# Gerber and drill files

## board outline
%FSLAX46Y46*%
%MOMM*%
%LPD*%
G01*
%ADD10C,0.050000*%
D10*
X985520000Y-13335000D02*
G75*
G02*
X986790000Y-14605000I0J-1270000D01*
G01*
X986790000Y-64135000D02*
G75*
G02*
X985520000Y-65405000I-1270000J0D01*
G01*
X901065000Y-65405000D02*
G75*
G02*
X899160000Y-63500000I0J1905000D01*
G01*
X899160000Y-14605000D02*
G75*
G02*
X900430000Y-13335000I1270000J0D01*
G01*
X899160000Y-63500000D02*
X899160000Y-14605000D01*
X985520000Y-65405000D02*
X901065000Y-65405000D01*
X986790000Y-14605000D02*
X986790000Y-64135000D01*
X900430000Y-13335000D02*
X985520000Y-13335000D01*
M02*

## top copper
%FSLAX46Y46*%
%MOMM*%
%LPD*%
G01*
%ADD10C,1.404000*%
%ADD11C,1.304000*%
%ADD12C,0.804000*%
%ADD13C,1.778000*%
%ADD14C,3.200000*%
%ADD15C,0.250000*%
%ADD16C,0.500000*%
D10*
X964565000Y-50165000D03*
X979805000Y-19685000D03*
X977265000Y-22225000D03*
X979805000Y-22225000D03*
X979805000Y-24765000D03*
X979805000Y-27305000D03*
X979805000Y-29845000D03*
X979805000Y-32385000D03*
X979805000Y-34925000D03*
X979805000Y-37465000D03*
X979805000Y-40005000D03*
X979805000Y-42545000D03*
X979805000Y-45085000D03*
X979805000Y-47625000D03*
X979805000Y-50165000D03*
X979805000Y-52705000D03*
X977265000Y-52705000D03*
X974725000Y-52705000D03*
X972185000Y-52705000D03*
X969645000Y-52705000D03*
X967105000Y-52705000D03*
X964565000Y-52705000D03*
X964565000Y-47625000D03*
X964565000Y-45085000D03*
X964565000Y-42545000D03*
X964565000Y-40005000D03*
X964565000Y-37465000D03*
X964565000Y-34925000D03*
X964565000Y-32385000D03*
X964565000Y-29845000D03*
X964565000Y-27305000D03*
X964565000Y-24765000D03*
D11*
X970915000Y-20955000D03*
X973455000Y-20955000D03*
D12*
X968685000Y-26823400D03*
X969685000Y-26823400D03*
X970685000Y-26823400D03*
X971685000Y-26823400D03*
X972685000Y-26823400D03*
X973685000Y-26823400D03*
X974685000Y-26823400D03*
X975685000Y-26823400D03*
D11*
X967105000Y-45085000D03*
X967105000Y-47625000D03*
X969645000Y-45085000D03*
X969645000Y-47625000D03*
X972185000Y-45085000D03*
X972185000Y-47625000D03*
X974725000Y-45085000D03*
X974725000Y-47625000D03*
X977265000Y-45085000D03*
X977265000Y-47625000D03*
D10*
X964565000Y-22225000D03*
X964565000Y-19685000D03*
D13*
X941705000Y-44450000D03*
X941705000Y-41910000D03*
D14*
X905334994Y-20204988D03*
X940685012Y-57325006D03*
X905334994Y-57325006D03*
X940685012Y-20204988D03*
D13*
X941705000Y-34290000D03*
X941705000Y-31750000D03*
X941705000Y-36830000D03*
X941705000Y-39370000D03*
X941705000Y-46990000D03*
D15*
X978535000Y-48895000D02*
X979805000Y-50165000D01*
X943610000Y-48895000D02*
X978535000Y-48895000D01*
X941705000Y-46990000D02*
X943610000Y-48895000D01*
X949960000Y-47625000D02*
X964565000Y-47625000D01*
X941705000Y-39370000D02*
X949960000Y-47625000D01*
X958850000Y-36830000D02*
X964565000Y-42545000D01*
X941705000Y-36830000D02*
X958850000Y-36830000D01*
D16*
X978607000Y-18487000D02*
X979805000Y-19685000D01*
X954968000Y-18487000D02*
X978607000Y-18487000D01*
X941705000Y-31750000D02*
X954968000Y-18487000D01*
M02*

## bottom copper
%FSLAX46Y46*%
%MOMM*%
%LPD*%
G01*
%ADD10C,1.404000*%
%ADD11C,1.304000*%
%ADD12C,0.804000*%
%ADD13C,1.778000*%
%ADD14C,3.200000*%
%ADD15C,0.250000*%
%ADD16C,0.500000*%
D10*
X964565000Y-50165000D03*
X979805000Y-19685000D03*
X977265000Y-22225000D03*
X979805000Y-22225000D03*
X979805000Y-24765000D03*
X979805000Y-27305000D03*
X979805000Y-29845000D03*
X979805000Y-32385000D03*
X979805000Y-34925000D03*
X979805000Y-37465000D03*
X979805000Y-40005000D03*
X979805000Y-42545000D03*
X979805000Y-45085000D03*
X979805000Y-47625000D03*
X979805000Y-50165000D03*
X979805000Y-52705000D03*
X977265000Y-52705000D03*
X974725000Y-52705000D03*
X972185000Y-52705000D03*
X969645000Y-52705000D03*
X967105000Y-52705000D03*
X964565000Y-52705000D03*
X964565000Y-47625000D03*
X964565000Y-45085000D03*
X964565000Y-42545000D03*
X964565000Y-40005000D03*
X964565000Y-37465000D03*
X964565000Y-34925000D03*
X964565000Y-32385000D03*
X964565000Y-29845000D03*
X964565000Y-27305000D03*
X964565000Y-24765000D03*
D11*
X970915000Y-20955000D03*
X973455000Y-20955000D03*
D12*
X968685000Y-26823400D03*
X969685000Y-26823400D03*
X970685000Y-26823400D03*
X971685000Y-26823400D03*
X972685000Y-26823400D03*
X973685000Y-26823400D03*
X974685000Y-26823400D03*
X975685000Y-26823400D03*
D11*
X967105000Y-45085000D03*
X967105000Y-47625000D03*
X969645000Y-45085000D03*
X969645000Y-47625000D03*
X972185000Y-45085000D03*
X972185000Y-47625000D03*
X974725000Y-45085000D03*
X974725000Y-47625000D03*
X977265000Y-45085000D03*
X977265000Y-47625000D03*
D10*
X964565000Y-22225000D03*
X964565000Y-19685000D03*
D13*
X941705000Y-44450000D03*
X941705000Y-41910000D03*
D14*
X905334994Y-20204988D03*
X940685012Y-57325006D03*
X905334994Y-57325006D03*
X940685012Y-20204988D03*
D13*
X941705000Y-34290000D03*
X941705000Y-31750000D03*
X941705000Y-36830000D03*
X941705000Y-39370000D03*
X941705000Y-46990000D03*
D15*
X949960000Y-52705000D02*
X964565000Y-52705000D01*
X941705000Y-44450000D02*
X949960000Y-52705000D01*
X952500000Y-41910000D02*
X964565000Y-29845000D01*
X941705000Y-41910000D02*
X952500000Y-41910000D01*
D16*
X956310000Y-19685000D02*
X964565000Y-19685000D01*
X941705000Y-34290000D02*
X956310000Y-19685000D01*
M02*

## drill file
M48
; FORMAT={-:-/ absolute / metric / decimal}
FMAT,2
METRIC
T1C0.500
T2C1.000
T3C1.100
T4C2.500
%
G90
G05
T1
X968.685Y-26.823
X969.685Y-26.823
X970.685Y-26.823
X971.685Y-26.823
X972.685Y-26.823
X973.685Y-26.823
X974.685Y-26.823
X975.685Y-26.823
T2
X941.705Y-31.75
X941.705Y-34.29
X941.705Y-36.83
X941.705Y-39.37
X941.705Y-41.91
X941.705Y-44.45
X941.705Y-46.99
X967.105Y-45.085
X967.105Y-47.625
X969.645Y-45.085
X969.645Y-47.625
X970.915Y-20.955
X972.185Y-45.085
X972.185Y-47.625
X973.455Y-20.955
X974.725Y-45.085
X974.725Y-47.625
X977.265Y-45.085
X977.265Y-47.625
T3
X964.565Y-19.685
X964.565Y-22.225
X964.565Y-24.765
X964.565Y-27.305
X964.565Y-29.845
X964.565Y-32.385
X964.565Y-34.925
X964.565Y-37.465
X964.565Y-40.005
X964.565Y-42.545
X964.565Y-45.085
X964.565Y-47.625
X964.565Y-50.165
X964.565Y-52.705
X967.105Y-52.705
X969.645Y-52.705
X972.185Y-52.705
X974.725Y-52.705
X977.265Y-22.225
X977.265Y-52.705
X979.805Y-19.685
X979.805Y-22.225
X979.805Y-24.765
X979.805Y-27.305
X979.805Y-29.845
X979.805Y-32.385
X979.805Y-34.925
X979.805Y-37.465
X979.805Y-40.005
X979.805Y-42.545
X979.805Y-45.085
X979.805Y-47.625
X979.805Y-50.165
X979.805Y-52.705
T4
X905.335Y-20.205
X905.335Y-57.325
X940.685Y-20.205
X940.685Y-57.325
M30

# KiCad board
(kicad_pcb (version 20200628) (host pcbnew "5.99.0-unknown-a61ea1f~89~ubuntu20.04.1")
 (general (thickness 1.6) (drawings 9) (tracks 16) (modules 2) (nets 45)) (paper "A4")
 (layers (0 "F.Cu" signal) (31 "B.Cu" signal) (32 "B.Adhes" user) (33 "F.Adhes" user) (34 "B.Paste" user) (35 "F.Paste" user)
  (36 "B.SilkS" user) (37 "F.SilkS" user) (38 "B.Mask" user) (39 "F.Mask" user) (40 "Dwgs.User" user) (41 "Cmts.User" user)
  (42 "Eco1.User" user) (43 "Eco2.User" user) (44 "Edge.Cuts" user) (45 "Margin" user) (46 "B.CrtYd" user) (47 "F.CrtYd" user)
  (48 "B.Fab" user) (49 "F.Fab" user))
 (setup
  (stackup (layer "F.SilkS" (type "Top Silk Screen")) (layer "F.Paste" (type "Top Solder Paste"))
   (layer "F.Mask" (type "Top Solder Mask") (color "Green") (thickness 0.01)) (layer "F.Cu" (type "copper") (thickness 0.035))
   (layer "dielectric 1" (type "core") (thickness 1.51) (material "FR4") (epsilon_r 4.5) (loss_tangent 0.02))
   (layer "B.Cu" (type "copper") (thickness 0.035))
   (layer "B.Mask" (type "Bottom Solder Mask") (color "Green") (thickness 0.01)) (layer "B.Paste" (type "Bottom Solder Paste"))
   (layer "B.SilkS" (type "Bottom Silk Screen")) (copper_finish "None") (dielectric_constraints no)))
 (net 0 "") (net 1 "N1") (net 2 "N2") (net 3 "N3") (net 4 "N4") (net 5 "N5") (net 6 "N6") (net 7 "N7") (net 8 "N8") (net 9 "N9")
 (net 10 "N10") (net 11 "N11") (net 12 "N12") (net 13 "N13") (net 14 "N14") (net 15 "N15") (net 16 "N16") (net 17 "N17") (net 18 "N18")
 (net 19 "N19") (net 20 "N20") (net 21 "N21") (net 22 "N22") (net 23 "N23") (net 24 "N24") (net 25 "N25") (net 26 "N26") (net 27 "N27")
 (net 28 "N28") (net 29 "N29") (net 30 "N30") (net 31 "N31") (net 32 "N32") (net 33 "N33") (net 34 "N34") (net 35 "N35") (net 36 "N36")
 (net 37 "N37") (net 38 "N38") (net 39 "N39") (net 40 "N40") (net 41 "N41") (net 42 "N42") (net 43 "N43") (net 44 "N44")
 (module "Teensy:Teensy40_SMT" (layer "F.Cu") (at 972.185 36.195 -90)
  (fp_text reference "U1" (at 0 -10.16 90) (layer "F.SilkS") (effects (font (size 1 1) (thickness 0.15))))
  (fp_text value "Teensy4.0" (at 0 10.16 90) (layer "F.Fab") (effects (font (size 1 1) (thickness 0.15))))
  (pad "13" thru_hole circle (at 13.97 7.62 270) (size 1.404 1.404) (drill 1.1) (layers *.Cu *.Mask) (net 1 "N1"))
  (pad "33" thru_hole circle (at -16.51 -7.62 270) (size 1.404 1.404) (drill 1.1) (layers *.Cu *.Mask) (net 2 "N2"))
  (pad "34" thru_hole circle (at -13.97 -5.08 270) (size 1.404 1.404) (drill 1.1) (layers *.Cu *.Mask) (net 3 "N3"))
  (pad "32" thru_hole circle (at -13.97 -7.62 270) (size 1.404 1.404) (drill 1.1) (layers *.Cu *.Mask) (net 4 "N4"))
  (pad "31" thru_hole circle (at -11.43 -7.62 270) (size 1.404 1.404) (drill 1.1) (layers *.Cu *.Mask) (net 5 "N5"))
  (pad "30" thru_hole circle (at -8.89 -7.62 270) (size 1.404 1.404) (drill 1.1) (layers *.Cu *.Mask) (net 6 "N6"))
  (pad "29" thru_hole circle (at -6.35 -7.62 270) (size 1.404 1.404) (drill 1.1) (layers *.Cu *.Mask) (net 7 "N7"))
  (pad "28" thru_hole circle (at -3.81 -7.62 270) (size 1.404 1.404) (drill 1.1) (layers *.Cu *.Mask) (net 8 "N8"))
  (pad "27" thru_hole circle (at -1.27 -7.62 270) (size 1.404 1.404) (drill 1.1) (layers *.Cu *.Mask) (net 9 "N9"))
  (pad "26" thru_hole circle (at 1.27 -7.62 270) (size 1.404 1.404) (drill 1.1) (layers *.Cu *.Mask) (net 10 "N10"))
  (pad "25" thru_hole circle (at 3.81 -7.62 270) (size 1.404 1.404) (drill 1.1) (layers *.Cu *.Mask) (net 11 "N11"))
  (pad "24" thru_hole circle (at 6.35 -7.62 270) (size 1.404 1.404) (drill 1.1) (layers *.Cu *.Mask) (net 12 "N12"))
  (pad "23" thru_hole circle (at 8.89 -7.62 270) (size 1.404 1.404) (drill 1.1) (layers *.Cu *.Mask) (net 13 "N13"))
  (pad "22" thru_hole circle (at 11.43 -7.62 270) (size 1.404 1.404) (drill 1.1) (layers *.Cu *.Mask) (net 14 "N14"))
  (pad "21" thru_hole circle (at 13.97 -7.62 270) (size 1.404 1.404) (drill 1.1) (layers *.Cu *.Mask) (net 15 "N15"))
  (pad "20" thru_hole circle (at 16.51 -7.62 270) (size 1.404 1.404) (drill 1.1) (layers *.Cu *.Mask) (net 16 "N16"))
  (pad "19" thru_hole circle (at 16.51 -5.08 270) (size 1.404 1.404) (drill 1.1) (layers *.Cu *.Mask) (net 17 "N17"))
  (pad "18" thru_hole circle (at 16.51 -2.54 270) (size 1.404 1.404) (drill 1.1) (layers *.Cu *.Mask) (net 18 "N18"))
  (pad "17" thru_hole circle (at 16.51 0 270) (size 1.404 1.404) (drill 1.1) (layers *.Cu *.Mask) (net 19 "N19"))
  (pad "16" thru_hole circle (at 16.51 2.54 270) (size 1.404 1.404) (drill 1.1) (layers *.Cu *.Mask) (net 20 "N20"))
  (pad "15" thru_hole circle (at 16.51 5.08 270) (size 1.404 1.404) (drill 1.1) (layers *.Cu *.Mask) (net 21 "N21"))
  (pad "14" thru_hole circle (at 16.51 7.62 270) (size 1.404 1.404) (drill 1.1) (layers *.Cu *.Mask) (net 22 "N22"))
  (pad "12" thru_hole circle (at 11.43 7.62 270) (size 1.404 1.404) (drill 1.1) (layers *.Cu *.Mask) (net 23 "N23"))
  (pad "11" thru_hole circle (at 8.89 7.62 270) (size 1.404 1.404) (drill 1.1) (layers *.Cu *.Mask) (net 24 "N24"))
  (pad "10" thru_hole circle (at 6.35 7.62 270) (size 1.404 1.404) (drill 1.1) (layers *.Cu *.Mask) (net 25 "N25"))
  (pad "9" thru_hole circle (at 3.81 7.62 270) (size 1.404 1.404) (drill 1.1) (layers *.Cu *.Mask) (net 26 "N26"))
  (pad "8" thru_hole circle (at 1.27 7.62 270) (size 1.404 1.404) (drill 1.1) (layers *.Cu *.Mask) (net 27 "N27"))
  (pad "7" thru_hole circle (at -1.27 7.62 270) (size 1.404 1.404) (drill 1.1) (layers *.Cu *.Mask) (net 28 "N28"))
  (pad "6" thru_hole circle (at -3.81 7.62 270) (size 1.404 1.404) (drill 1.1) (layers *.Cu *.Mask) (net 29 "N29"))
  (pad "5" thru_hole circle (at -6.35 7.62 270) (size 1.404 1.404) (drill 1.1) (layers *.Cu *.Mask) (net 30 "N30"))
  (pad "4" thru_hole circle (at -8.89 7.62 270) (size 1.404 1.404) (drill 1.1) (layers *.Cu *.Mask) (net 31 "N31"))
  (pad "3" thru_hole circle (at -11.43 7.62 270) (size 1.404 1.404) (drill 1.1) (layers *.Cu *.Mask) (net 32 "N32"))
  (pad "54" thru_hole circle (at -15.24 1.27 270) (size 1.304 1.304) (drill 1) (layers *.Cu *.Mask))
  (pad "53" thru_hole circle (at -15.24 -1.27 270) (size 1.304 1.304) (drill 1) (layers *.Cu *.Mask))
  (pad "52" thru_hole circle (at -9.3716 3.5 270) (size 0.804 0.804) (drill 0.5) (layers *.Cu *.Mask))
  (pad "51" thru_hole circle (at -9.3716 2.5 270) (size 0.804 0.804) (drill 0.5) (layers *.Cu *.Mask))
  (pad "50" thru_hole circle (at -9.3716 1.5 270) (size 0.804 0.804) (drill 0.5) (layers *.Cu *.Mask))
  (pad "49" thru_hole circle (at -9.3716 0.5 270) (size 0.804 0.804) (drill 0.5) (layers *.Cu *.Mask))
  (pad "48" thru_hole circle (at -9.3716 -0.5 270) (size 0.804 0.804) (drill 0.5) (layers *.Cu *.Mask))
  (pad "47" thru_hole circle (at -9.3716 -1.5 270) (size 0.804 0.804) (drill 0.5) (layers *.Cu *.Mask))
  (pad "46" thru_hole circle (at -9.3716 -2.5 270) (size 0.804 0.804) (drill 0.5) (layers *.Cu *.Mask))
  (pad "45" thru_hole circle (at -9.3716 -3.5 270) (size 0.804 0.804) (drill 0.5) (layers *.Cu *.Mask))
  (pad "44" thru_hole circle (at 8.89 5.08 270) (size 1.304 1.304) (drill 1) (layers *.Cu *.Mask) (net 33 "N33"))
  (pad "43" thru_hole circle (at 11.43 5.08 270) (size 1.304 1.304) (drill 1) (layers *.Cu *.Mask) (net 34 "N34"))
  (pad "42" thru_hole circle (at 8.89 2.54 270) (size 1.304 1.304) (drill 1) (layers *.Cu *.Mask) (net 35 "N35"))
  (pad "41" thru_hole circle (at 11.43 2.54 270) (size 1.304 1.304) (drill 1) (layers *.Cu *.Mask) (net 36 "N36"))
  (pad "40" thru_hole circle (at 8.89 0 270) (size 1.304 1.304) (drill 1) (layers *.Cu *.Mask) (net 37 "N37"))
  (pad "39" thru_hole circle (at 11.43 0 270) (size 1.304 1.304) (drill 1) (layers *.Cu *.Mask) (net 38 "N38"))
  (pad "38" thru_hole circle (at 8.89 -2.54 270) (size 1.304 1.304) (drill 1) (layers *.Cu *.Mask) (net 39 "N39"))
  (pad "37" thru_hole circle (at 11.43 -2.54 270) (size 1.304 1.304) (drill 1) (layers *.Cu *.Mask) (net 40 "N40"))
  (pad "36" thru_hole circle (at 8.89 -5.08 270) (size 1.304 1.304) (drill 1) (layers *.Cu *.Mask) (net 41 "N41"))
  (pad "35" thru_hole circle (at 11.43 -5.08 270) (size 1.304 1.304) (drill 1) (layers *.Cu *.Mask) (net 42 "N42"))
  (pad "2" thru_hole circle (at -13.97 7.62 270) (size 1.404 1.404) (drill 1.1) (layers *.Cu *.Mask) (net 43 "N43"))
  (pad "1" thru_hole circle (at -16.51 7.62 270) (size 1.404 1.404) (drill 1.1) (layers *.Cu *.Mask) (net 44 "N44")))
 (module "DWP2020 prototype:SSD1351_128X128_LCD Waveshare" (layer "F.Cu") (at 921.385 37.465)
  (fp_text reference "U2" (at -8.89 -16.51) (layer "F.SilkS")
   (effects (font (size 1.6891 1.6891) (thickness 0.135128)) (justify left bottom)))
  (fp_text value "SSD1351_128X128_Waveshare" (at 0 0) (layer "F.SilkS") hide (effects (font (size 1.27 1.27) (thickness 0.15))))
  (pad "JP1$6" thru_hole circle (at 20.32 6.985 90) (size 1.778 1.778) (drill 1) (layers *.Cu *.Mask) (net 22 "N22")
   (solder_mask_margin 0.1016))
  (pad "JP1$5" thru_hole circle (at 20.32 4.445 90) (size 1.778 1.778) (drill 1) (layers *.Cu *.Mask) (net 30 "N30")
   (solder_mask_margin 0.1016))
  (pad "U$26$P$1" thru_hole circle (at -16.050006 -17.260012) (size 3.2 3.2) (drill 2.5) (layers *.Cu *.Mask) (solder_mask_margin 0.1016))
  (pad "U$25$P$1" thru_hole circle (at 19.300012 19.860006) (size 3.2 3.2) (drill 2.5) (layers *.Cu *.Mask) (solder_mask_margin 0.1016))
  (pad "U$24$P$1" thru_hole circle (at -16.050006 19.860006) (size 3.2 3.2) (drill 2.5) (layers *.Cu *.Mask) (solder_mask_margin 0.1016))
  (pad "U$23$P$1" thru_hole circle (at 19.300012 -17.260012) (size 3.2 3.2) (drill 2.5) (layers *.Cu *.Mask) (solder_mask_margin 0.1016))
  (pad "JP1$2" thru_hole circle (at 20.32 -3.175 90) (size 1.778 1.778) (drill 1) (layers *.Cu *.Mask) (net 44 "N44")
   (solder_mask_margin 0.1016))
  (pad "JP1$1" thru_hole circle (at 20.32 -5.715 90) (size 1.778 1.778) (drill 1) (layers *.Cu *.Mask) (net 2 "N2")
   (solder_mask_margin 0.1016))
  (pad "JP1$3" thru_hole circle (at 20.32 -0.635 90) (size 1.778 1.778) (drill 1) (layers *.Cu *.Mask) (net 25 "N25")
   (solder_mask_margin 0.1016))
  (pad "JP1$4" thru_hole circle (at 20.32 1.905 90) (size 1.778 1.778) (drill 1) (layers *.Cu *.Mask) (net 23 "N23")
   (solder_mask_margin 0.1016))
  (pad "JP1$7" thru_hole circle (at 20.32 9.525 90) (size 1.778 1.778) (drill 1) (layers *.Cu *.Mask) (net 15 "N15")
   (solder_mask_margin 0.1016)))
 (gr_arc (start 985.52 14.605) (end 986.79 14.605) (angle -90) (layer "Edge.Cuts") (width 0.05))
 (gr_arc (start 985.52 64.135) (end 985.52 65.405) (angle -90) (layer "Edge.Cuts") (width 0.05))
 (gr_arc (start 901.065 63.5) (end 899.16 63.5) (angle -90) (layer "Edge.Cuts") (width 0.05))
 (gr_arc (start 900.43 14.605) (end 900.43 13.335) (angle -90) (layer "Edge.Cuts") (width 0.05))
 (gr_line (start 899.16 63.5) (end 899.16 14.605) (layer "Edge.Cuts") (width 0.05))
 (gr_line (start 985.52 65.405) (end 901.065 65.405) (layer "Edge.Cuts") (width 0.05))
 (gr_line (start 986.79 14.605) (end 986.79 64.135) (layer "Edge.Cuts") (width 0.05))
 (gr_line (start 900.43 13.335) (end 985.52 13.335) (layer "Edge.Cuts") (width 0.05))
 (segment (start 949.96 52.705) (end 964.565 52.705) (width 0.25) (layer "B.Cu") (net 22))
 (segment (start 941.705 44.45) (end 949.96 52.705) (width 0.25) (layer "B.Cu") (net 22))
 (segment (start 978.535 48.895) (end 979.805 50.165) (width 0.25) (layer "F.Cu") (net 15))
 (segment (start 943.61 48.895) (end 978.535 48.895) (width 0.25) (layer "F.Cu") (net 15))
 (segment (start 941.705 46.99) (end 943.61 48.895) (width 0.25) (layer "F.Cu") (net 15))
 (segment (start 949.96 47.625) (end 964.565 47.625) (width 0.25) (layer "F.Cu") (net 23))
 (segment (start 941.705 39.37) (end 949.96 47.625) (width 0.25) (layer "F.Cu") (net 23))
 (segment (start 958.85 36.83) (end 964.565 42.545) (width 0.25) (layer "F.Cu") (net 25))
 (segment (start 941.705 36.83) (end 958.85 36.83) (width 0.25) (layer "F.Cu") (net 25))
 (segment (start 952.5 41.91) (end 964.565 29.845) (width 0.25) (layer "B.Cu") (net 30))
 (segment (start 941.705 41.91) (end 952.5 41.91) (width 0.25) (layer "B.Cu") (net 30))
 (segment (start 956.31 19.685) (end 964.565 19.685) (width 0.5) (layer "B.Cu") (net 44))
 (segment (start 941.705 34.29) (end 956.31 19.685) (width 0.5) (layer "B.Cu") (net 44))
 (segment (start 978.607 18.487) (end 979.805 19.685) (width 0.5) (layer "F.Cu") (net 2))
 (segment (start 954.968 18.487) (end 978.607 18.487) (width 0.5) (layer "F.Cu") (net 2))
 (segment (start 941.705 31.75) (end 954.968 18.487) (width 0.5) (layer "F.Cu") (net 2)))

